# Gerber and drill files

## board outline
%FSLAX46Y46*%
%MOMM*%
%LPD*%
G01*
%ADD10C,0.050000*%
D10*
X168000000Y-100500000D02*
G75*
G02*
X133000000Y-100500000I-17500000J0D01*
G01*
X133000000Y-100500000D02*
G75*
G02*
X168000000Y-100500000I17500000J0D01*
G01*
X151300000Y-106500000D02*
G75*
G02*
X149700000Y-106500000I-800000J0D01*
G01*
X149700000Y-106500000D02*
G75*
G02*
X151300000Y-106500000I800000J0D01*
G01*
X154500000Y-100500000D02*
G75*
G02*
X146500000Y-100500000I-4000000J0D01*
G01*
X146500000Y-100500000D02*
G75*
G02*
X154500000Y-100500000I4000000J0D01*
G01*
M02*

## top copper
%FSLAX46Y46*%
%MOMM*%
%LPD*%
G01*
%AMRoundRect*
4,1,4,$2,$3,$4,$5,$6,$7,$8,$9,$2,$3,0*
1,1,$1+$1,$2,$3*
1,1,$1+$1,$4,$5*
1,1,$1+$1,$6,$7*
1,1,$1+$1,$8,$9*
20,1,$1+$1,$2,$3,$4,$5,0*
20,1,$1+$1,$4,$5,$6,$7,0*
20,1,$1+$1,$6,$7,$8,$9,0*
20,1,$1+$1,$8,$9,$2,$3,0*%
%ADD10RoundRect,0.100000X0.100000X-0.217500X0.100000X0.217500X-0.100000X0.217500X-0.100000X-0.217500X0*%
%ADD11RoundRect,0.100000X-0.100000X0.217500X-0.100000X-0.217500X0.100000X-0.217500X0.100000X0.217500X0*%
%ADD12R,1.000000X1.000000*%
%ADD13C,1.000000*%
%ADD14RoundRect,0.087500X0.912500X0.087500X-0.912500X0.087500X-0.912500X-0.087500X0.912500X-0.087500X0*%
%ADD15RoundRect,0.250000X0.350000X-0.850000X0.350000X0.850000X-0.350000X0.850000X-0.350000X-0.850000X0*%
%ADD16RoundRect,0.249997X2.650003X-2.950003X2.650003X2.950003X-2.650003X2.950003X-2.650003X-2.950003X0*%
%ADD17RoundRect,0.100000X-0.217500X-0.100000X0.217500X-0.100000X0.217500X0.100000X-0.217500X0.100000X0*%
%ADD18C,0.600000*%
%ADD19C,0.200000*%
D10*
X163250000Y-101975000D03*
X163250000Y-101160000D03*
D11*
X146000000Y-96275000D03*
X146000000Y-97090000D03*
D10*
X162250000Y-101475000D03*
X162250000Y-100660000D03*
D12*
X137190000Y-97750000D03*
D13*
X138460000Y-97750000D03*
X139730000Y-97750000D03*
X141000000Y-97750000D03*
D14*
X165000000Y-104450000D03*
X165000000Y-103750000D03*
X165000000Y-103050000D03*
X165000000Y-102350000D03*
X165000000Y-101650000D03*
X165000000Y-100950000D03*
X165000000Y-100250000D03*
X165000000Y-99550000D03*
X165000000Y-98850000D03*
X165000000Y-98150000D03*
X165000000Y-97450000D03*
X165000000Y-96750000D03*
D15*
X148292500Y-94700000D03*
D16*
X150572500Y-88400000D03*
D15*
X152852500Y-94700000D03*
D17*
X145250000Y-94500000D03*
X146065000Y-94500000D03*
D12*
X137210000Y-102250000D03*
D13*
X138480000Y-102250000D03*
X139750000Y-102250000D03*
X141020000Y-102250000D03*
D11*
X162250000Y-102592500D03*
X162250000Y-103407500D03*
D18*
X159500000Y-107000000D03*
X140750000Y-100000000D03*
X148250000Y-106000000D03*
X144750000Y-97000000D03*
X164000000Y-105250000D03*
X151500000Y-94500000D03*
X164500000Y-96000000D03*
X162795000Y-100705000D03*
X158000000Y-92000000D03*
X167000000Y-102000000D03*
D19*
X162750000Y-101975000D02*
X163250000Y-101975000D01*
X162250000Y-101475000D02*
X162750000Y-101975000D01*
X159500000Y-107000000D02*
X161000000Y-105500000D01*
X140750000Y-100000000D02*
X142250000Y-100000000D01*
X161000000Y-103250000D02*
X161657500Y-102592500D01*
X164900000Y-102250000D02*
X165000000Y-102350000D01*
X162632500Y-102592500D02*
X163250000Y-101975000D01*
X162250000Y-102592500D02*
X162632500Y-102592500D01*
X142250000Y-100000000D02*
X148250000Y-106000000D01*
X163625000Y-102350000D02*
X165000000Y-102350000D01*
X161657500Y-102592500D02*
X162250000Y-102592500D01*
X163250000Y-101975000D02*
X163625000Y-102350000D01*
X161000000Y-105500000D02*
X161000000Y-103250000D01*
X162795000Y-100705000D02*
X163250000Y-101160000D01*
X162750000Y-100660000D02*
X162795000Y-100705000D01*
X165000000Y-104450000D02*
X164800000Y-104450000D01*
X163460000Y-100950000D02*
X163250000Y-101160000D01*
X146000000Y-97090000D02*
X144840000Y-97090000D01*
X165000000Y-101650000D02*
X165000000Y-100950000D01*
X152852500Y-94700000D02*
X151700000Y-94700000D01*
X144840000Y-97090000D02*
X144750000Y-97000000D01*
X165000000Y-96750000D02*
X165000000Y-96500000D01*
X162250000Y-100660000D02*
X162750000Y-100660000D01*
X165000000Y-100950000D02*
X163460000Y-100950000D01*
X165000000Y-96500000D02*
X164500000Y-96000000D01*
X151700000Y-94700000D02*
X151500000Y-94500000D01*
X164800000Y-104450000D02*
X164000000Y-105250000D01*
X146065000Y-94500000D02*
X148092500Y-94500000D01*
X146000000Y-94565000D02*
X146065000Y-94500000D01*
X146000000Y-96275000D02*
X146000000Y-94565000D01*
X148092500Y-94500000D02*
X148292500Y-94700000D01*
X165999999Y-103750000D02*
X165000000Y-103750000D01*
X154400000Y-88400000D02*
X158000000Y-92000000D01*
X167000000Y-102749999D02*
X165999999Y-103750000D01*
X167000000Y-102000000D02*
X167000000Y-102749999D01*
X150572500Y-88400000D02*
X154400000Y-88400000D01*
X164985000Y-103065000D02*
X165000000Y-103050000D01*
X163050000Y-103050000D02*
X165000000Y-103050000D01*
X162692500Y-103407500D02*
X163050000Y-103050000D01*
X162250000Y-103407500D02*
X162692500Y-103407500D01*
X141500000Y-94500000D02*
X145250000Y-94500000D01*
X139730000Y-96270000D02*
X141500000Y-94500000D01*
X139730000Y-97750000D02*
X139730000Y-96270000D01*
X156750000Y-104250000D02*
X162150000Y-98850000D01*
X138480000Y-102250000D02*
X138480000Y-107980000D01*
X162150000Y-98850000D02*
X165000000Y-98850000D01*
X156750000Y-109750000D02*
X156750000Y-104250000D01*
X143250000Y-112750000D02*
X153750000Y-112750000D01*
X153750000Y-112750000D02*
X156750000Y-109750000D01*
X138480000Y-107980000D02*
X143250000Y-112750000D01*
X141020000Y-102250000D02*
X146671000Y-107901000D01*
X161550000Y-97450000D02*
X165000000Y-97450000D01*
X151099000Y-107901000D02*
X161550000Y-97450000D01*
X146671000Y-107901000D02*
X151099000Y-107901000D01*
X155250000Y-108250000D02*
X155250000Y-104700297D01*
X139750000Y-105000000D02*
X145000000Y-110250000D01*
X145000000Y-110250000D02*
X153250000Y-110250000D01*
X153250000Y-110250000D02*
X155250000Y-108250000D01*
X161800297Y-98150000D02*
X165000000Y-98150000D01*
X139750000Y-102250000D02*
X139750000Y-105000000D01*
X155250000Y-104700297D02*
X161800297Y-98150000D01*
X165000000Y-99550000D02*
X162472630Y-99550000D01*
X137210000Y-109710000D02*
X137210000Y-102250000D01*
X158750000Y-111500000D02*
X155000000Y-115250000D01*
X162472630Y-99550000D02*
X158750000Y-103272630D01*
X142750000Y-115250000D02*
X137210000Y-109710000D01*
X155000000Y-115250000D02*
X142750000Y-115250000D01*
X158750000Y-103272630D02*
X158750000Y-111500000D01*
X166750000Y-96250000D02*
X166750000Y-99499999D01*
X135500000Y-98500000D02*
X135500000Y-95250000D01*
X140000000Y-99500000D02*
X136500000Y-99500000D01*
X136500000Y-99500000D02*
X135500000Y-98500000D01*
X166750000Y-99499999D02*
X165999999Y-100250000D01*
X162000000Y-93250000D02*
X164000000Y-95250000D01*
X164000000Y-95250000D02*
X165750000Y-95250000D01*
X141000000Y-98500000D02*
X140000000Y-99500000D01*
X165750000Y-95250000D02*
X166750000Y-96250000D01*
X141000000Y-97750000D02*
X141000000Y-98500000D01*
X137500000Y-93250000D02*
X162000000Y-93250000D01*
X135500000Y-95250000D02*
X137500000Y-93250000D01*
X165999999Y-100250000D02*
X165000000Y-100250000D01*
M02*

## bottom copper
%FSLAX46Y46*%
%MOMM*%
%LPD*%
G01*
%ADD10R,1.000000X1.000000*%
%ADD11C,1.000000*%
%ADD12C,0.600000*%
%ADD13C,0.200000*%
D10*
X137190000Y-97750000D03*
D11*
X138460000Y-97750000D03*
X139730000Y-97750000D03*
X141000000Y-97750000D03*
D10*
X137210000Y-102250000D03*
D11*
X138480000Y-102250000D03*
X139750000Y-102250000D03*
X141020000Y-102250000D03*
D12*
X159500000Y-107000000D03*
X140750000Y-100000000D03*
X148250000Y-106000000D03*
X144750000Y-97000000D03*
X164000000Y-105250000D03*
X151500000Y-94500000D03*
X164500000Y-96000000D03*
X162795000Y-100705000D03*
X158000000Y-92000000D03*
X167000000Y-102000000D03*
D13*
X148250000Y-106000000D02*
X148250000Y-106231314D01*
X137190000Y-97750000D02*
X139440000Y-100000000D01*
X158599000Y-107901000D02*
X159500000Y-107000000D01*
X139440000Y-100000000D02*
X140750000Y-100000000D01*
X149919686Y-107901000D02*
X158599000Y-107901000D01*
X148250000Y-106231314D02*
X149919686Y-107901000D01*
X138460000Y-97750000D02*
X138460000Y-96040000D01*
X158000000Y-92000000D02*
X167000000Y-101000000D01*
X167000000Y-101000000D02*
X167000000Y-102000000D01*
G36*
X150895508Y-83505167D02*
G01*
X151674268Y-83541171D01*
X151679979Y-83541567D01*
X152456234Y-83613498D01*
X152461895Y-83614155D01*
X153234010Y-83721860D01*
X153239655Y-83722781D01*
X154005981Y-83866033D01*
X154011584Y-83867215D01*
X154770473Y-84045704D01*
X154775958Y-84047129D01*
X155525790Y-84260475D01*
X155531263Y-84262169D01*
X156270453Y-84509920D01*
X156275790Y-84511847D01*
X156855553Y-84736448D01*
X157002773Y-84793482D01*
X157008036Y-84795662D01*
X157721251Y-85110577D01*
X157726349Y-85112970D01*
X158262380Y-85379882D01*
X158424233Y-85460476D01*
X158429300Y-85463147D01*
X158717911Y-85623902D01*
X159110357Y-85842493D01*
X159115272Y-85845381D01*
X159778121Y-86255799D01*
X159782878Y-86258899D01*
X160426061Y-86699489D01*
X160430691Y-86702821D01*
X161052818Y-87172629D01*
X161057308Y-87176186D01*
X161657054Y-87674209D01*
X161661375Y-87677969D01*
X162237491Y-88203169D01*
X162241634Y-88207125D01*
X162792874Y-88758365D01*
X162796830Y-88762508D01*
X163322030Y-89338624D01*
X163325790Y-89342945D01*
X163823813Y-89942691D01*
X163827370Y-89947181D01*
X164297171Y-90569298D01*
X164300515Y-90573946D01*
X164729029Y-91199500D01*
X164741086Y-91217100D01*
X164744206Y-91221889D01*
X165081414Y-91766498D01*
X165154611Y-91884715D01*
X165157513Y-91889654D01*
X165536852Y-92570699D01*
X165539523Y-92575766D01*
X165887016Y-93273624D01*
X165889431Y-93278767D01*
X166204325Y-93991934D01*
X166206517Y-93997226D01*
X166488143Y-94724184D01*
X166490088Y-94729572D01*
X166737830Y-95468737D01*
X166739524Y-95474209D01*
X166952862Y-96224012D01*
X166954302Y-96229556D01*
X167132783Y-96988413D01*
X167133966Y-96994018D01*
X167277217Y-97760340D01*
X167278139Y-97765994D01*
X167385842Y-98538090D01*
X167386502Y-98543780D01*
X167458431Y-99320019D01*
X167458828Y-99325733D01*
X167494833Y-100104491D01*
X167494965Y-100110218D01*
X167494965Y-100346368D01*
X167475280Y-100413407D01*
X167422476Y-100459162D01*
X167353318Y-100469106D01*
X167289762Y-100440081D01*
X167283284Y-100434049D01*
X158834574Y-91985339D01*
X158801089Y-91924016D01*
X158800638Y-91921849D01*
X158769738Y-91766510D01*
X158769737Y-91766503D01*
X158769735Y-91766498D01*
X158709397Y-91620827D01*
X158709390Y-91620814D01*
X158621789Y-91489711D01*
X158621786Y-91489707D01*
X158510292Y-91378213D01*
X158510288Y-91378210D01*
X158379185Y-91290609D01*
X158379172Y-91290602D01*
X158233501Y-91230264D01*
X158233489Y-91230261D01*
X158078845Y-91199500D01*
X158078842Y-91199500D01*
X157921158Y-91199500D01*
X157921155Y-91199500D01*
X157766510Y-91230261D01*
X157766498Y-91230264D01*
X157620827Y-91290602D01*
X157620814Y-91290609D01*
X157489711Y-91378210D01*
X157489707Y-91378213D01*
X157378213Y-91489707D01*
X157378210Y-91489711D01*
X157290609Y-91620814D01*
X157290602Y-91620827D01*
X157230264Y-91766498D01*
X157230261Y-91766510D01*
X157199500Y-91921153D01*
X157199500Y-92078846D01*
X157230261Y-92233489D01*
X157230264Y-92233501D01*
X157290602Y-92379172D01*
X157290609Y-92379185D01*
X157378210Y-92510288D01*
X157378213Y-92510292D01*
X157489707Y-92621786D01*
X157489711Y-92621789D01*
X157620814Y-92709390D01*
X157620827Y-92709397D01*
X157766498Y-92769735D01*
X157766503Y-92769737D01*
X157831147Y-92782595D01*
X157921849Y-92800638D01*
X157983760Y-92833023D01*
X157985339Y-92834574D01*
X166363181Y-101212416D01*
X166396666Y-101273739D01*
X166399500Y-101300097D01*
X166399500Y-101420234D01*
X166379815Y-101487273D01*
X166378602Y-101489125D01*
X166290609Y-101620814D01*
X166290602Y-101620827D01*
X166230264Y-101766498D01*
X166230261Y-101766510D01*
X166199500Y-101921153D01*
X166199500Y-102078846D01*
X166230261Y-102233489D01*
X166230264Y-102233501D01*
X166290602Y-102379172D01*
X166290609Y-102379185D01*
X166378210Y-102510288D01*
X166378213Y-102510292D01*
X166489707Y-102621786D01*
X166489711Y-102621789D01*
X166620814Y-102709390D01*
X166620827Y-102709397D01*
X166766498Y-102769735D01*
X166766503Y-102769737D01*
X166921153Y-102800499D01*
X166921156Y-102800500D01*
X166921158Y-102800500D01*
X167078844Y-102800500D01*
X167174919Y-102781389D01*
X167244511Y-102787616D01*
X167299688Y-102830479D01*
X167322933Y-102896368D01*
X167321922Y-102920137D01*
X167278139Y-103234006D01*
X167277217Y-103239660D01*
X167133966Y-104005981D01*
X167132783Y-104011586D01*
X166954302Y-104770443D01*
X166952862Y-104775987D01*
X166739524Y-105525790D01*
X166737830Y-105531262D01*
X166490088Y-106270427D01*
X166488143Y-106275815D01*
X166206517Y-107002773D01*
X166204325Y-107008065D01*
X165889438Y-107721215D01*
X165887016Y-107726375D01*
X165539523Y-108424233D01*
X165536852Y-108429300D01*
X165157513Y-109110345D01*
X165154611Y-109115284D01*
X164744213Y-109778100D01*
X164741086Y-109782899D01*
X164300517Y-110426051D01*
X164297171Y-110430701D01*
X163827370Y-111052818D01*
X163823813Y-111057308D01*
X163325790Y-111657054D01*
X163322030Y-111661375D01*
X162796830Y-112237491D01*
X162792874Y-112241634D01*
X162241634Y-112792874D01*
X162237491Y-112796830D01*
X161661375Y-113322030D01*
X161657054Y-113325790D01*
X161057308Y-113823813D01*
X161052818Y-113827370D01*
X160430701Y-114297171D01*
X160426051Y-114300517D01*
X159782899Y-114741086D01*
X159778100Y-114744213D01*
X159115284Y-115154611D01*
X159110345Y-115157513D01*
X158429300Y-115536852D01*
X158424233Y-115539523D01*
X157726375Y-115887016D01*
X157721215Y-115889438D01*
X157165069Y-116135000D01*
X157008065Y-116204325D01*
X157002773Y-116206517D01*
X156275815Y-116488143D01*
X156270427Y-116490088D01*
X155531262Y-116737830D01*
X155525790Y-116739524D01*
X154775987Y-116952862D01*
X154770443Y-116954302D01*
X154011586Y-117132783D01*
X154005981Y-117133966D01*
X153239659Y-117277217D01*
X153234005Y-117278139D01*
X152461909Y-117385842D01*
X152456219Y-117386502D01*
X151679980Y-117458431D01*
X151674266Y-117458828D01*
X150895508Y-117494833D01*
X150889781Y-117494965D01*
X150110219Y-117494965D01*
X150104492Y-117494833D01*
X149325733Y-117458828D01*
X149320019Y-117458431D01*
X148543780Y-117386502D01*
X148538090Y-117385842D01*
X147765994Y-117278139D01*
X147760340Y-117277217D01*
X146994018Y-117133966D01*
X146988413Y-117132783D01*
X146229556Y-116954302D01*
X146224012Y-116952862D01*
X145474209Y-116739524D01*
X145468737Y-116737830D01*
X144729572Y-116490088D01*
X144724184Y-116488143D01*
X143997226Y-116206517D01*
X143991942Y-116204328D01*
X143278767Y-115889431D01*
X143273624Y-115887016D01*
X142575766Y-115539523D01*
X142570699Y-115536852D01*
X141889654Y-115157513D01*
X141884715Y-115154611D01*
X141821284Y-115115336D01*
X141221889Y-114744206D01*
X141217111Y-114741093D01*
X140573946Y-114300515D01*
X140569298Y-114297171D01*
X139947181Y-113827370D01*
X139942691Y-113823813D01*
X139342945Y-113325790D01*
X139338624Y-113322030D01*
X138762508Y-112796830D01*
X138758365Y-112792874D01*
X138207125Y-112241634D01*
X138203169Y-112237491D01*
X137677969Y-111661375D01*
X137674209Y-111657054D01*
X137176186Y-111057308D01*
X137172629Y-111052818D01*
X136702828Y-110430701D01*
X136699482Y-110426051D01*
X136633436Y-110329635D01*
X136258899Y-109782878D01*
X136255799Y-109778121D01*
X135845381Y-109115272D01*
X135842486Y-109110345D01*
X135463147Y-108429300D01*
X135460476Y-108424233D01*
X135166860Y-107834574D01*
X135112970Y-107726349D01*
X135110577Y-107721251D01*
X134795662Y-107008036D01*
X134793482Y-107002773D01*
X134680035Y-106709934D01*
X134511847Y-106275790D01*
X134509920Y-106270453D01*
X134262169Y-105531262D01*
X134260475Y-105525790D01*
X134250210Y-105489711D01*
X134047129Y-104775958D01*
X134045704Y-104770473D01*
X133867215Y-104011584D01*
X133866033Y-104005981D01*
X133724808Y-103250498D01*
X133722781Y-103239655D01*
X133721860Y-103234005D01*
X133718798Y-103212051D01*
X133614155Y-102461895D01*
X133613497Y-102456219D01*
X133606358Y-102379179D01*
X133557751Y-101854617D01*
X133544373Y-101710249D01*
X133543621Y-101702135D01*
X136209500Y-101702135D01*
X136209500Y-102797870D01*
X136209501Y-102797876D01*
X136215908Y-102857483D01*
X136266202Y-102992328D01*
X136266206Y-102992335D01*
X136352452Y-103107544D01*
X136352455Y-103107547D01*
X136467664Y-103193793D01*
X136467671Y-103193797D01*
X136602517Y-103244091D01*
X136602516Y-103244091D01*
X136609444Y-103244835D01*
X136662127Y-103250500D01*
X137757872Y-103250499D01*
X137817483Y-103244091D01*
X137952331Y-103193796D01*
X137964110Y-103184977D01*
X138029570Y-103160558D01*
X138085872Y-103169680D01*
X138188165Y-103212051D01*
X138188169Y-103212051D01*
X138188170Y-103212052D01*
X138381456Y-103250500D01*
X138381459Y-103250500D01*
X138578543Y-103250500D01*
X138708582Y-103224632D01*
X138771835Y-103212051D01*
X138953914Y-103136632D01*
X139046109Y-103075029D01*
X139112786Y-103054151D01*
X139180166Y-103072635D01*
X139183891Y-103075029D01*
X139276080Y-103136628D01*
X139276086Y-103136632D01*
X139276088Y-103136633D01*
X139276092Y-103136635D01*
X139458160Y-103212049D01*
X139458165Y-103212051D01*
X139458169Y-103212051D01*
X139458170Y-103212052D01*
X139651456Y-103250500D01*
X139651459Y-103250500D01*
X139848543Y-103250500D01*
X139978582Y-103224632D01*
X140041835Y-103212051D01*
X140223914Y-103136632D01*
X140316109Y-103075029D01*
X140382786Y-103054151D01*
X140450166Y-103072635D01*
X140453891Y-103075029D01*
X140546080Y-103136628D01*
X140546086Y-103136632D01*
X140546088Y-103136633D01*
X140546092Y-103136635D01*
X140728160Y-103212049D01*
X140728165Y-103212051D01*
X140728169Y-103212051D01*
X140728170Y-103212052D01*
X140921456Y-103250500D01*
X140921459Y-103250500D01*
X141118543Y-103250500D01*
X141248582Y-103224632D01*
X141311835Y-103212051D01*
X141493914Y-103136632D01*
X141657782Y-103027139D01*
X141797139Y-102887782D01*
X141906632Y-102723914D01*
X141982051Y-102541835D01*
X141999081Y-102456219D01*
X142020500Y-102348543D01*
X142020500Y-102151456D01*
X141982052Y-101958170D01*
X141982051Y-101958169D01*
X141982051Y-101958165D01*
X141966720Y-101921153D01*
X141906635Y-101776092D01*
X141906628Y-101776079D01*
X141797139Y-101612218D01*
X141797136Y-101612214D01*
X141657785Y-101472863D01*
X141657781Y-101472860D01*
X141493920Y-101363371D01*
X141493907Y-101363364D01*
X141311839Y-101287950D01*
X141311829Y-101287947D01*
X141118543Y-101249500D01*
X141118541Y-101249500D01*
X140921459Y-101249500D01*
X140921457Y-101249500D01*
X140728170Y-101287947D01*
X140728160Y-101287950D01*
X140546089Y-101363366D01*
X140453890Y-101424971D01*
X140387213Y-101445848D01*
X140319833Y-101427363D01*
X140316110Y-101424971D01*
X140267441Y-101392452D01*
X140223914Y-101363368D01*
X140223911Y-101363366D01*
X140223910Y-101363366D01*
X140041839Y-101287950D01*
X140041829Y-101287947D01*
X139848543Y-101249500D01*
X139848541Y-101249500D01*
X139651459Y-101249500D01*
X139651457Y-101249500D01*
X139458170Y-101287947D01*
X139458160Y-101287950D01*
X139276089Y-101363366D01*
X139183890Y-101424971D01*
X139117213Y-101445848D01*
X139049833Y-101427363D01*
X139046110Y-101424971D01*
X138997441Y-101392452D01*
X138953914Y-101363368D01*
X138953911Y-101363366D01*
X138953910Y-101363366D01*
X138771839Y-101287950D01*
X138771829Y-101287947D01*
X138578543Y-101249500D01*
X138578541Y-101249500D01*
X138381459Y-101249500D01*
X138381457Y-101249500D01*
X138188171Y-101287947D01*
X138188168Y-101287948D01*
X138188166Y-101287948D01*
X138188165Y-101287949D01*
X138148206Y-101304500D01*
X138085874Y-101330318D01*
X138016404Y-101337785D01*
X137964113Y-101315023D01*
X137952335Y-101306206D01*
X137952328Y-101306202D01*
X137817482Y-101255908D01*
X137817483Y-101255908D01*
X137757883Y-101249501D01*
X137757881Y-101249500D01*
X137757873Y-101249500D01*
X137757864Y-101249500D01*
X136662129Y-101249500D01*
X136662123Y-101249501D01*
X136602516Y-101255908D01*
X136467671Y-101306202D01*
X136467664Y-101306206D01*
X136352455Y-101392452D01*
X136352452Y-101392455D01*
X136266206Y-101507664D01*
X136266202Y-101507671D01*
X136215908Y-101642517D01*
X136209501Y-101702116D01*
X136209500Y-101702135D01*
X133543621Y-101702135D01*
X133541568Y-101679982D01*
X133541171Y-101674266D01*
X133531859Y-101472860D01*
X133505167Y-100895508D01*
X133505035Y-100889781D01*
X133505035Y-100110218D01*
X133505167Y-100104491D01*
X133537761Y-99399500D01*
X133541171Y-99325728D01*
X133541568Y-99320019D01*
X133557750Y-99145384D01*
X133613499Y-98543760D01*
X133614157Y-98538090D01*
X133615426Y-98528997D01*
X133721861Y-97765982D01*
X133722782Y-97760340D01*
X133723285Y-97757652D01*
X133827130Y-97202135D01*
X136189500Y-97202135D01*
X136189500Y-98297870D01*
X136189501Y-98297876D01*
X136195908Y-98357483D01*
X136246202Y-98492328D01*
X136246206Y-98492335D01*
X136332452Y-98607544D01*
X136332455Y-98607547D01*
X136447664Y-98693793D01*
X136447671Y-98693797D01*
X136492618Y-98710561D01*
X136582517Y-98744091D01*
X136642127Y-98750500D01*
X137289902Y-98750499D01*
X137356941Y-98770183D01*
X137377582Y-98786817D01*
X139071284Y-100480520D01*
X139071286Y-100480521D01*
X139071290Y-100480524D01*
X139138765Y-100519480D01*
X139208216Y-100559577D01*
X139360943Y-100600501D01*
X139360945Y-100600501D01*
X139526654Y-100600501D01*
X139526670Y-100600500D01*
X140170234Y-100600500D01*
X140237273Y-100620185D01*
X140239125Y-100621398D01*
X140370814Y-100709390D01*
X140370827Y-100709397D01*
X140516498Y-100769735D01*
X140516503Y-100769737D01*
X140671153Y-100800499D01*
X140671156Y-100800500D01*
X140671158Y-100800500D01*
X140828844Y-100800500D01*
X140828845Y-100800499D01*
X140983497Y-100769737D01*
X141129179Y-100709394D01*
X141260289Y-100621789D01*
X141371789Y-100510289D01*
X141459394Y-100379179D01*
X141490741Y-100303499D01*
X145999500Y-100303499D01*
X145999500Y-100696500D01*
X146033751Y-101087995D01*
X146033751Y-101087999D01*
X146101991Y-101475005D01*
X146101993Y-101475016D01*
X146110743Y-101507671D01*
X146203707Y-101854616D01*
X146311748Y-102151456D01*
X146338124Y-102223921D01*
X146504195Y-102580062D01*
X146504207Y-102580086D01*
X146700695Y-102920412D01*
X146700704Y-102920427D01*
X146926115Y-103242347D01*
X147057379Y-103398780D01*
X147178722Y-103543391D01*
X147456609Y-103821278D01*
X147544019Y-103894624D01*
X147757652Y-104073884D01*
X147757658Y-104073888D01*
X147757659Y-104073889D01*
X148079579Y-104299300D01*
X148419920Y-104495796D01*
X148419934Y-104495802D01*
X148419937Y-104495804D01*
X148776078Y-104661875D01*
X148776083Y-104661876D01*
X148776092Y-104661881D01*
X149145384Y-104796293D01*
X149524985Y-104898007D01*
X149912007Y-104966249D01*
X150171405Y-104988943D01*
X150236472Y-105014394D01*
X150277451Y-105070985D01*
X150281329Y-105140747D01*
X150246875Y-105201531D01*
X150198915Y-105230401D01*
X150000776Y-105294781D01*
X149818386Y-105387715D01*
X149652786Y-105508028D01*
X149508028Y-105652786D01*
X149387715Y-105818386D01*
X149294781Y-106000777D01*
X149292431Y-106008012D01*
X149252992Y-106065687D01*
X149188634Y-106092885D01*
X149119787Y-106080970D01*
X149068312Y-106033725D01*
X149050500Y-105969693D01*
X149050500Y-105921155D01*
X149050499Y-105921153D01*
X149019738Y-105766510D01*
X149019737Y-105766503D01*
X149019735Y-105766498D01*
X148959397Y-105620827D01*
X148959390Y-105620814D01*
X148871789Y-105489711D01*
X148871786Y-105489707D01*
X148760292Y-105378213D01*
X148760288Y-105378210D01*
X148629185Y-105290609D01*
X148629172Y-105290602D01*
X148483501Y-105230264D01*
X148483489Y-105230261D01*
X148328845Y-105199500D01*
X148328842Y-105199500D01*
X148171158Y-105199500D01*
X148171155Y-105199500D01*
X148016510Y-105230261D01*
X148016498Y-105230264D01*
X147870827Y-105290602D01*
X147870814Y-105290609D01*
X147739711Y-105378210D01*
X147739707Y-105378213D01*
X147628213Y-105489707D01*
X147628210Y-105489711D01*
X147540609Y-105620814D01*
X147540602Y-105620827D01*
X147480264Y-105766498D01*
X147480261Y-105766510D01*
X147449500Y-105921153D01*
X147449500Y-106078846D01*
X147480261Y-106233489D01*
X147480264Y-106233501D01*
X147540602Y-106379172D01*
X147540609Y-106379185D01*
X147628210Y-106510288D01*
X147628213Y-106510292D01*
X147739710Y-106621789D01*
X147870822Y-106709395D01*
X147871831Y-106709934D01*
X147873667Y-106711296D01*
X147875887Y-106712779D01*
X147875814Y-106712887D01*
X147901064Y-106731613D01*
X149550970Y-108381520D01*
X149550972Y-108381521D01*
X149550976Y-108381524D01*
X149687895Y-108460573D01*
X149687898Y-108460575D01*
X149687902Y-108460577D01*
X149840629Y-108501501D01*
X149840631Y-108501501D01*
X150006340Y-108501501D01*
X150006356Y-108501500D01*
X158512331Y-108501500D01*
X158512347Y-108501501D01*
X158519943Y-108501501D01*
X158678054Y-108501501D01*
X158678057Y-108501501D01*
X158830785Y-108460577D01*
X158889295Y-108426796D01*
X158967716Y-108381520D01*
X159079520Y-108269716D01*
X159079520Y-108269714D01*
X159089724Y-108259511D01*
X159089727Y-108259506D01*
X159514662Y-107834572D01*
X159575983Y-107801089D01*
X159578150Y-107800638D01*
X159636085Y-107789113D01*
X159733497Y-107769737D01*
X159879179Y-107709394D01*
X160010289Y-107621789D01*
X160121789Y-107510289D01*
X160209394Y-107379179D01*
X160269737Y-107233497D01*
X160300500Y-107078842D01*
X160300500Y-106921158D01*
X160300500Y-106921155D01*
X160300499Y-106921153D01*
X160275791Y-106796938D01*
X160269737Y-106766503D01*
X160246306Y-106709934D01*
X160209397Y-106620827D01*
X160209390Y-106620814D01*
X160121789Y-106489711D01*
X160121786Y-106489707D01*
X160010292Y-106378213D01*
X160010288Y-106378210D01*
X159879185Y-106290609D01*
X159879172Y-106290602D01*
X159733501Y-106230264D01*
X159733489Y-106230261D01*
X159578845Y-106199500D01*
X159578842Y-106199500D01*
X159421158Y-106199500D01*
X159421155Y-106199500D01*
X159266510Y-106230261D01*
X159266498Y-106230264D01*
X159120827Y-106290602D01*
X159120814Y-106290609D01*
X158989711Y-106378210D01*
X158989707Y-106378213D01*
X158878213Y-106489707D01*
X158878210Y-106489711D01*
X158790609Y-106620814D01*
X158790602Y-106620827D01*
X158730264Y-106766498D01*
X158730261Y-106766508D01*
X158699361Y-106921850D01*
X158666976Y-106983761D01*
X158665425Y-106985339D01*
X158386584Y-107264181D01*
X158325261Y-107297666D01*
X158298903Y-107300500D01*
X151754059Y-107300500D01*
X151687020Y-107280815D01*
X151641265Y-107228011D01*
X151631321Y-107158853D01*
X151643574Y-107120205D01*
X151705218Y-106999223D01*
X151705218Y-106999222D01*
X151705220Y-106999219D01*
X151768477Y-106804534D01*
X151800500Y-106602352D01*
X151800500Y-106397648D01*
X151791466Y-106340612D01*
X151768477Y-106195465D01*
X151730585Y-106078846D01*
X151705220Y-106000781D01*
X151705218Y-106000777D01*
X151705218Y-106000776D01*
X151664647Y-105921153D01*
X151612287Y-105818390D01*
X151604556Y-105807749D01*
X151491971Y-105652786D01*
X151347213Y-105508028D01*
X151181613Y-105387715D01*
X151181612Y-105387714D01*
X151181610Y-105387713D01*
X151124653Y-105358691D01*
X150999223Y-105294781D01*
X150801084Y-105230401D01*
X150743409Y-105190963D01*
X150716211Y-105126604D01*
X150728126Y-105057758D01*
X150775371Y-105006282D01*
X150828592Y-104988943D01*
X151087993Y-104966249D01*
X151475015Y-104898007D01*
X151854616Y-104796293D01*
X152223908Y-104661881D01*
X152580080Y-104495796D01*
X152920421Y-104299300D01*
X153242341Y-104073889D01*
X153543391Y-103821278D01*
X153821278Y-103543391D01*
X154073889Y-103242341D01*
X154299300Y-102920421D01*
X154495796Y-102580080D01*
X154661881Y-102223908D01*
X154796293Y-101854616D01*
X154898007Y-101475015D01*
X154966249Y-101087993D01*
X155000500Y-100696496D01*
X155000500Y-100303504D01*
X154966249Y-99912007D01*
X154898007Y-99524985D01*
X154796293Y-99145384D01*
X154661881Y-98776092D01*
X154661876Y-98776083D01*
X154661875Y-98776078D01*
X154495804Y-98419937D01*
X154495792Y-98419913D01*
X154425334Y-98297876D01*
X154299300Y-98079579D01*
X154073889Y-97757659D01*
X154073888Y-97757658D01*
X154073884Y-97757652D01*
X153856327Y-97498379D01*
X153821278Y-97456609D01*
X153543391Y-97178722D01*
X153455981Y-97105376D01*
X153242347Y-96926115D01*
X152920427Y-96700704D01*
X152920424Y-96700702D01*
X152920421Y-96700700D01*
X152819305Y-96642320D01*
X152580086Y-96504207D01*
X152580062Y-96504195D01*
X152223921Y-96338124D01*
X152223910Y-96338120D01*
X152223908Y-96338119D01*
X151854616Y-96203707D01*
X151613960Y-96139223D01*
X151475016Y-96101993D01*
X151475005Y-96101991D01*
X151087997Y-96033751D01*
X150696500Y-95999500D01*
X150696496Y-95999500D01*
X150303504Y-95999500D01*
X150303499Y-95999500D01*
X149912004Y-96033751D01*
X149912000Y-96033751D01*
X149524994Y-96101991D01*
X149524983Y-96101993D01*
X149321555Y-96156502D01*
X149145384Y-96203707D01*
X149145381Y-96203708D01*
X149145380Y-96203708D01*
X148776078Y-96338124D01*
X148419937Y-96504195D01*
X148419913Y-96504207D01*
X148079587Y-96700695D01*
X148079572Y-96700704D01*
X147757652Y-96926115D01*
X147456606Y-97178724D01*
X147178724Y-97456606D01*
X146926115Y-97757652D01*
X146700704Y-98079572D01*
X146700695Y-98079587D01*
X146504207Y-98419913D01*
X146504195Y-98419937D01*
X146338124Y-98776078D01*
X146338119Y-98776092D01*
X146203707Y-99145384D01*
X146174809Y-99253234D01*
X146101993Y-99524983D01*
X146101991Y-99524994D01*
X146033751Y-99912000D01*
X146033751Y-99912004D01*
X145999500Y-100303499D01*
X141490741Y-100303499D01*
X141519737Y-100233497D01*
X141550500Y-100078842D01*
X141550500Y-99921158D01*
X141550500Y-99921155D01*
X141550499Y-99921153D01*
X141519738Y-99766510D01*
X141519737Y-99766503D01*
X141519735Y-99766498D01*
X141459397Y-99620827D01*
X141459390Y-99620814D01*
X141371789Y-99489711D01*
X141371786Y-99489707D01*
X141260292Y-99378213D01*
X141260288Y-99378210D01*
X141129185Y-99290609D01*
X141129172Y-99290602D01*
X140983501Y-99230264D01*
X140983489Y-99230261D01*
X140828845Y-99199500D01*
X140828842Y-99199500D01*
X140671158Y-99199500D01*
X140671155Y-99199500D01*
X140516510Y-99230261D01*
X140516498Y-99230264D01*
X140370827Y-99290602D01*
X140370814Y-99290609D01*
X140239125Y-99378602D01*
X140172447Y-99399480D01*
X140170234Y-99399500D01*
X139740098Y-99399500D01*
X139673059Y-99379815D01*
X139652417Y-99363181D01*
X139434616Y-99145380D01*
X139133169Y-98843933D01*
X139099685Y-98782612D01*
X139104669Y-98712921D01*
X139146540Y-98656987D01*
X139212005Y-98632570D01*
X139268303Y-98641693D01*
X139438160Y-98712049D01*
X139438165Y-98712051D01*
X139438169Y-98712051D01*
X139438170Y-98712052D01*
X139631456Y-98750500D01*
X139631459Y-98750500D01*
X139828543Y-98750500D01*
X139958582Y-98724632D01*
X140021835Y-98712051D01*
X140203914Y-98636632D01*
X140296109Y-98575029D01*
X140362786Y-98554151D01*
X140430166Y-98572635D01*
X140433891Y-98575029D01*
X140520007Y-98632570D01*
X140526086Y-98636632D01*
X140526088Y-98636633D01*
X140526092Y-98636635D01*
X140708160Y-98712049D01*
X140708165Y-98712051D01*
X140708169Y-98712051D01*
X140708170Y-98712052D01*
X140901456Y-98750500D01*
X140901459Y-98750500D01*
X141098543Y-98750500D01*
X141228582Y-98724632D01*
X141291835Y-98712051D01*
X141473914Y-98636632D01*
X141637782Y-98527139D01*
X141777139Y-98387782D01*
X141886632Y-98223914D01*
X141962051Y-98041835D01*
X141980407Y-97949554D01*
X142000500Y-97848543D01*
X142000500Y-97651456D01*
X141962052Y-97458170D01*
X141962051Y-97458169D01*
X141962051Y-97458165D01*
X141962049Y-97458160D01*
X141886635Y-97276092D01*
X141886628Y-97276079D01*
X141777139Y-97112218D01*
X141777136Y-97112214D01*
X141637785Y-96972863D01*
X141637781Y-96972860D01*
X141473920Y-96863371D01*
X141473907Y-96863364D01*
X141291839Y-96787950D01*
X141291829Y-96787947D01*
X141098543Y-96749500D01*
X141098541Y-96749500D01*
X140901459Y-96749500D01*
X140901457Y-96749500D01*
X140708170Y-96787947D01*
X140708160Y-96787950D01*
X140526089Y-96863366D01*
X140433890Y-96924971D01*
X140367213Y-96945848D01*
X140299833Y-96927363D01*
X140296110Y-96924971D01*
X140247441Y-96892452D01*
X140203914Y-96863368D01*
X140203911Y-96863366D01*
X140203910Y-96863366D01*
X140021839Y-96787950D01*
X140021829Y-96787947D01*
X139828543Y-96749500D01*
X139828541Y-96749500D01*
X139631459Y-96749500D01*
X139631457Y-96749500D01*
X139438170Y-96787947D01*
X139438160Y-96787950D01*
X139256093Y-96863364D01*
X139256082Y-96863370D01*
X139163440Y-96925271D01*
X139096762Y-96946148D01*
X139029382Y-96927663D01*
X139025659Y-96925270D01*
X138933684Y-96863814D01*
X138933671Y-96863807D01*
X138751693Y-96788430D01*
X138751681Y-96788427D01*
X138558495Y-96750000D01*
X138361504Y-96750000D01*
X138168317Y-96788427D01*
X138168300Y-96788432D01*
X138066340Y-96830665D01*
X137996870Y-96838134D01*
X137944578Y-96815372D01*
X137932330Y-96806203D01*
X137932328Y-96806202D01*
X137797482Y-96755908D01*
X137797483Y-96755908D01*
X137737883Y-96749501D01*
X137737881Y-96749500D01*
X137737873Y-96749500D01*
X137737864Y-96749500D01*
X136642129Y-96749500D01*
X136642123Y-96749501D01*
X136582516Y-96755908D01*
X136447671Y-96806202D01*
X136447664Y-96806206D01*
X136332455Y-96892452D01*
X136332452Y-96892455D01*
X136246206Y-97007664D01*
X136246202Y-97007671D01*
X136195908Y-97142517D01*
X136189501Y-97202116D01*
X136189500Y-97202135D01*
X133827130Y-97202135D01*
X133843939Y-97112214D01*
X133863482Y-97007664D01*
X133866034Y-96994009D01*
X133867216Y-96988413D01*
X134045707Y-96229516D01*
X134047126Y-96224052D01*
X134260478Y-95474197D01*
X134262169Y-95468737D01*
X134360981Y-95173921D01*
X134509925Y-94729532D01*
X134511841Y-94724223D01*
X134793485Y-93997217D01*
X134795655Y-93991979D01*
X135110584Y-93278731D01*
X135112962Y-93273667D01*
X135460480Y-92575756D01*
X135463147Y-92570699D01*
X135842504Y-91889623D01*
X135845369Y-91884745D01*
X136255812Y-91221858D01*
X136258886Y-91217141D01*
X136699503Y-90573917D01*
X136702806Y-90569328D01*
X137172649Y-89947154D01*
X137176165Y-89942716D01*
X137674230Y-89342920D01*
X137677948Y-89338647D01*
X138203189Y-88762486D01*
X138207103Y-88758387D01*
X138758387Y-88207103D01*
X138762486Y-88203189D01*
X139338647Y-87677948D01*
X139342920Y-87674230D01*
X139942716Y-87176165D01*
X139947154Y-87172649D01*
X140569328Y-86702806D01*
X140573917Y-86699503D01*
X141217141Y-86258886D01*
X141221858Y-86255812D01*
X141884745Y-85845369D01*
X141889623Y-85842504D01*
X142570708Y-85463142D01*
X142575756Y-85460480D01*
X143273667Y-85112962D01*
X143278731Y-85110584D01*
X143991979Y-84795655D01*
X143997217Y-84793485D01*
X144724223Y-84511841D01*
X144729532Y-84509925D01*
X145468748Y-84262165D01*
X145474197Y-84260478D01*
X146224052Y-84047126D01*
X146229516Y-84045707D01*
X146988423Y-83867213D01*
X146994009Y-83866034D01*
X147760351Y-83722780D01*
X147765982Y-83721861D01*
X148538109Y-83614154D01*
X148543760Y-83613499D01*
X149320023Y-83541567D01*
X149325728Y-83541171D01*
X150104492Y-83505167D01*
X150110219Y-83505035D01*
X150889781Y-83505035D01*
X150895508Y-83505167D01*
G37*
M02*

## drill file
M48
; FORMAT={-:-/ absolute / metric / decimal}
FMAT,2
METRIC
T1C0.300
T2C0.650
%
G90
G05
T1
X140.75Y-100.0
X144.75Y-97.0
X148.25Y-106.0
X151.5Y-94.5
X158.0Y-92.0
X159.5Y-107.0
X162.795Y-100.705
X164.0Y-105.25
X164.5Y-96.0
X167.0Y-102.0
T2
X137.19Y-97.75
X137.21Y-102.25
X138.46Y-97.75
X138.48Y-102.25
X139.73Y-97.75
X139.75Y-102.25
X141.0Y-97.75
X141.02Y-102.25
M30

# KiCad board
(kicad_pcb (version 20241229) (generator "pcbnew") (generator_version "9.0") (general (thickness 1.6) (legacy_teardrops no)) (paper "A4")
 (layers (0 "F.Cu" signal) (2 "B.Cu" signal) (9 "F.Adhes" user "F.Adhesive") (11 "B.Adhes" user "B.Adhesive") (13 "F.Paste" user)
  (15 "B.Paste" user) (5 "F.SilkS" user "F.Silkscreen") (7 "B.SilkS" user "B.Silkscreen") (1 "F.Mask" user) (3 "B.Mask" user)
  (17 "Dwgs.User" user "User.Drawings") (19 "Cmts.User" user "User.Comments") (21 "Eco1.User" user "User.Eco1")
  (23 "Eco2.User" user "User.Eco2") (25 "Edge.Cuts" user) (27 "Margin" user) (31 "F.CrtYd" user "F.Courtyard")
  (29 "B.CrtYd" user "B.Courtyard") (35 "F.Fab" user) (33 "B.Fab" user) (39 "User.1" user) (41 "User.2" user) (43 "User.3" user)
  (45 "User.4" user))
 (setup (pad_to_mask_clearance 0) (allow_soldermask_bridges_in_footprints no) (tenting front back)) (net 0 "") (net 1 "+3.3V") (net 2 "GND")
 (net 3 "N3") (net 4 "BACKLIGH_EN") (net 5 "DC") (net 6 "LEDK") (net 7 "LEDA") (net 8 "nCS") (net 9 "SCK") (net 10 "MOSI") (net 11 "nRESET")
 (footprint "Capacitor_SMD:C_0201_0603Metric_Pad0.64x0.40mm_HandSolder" (layer "F.Cu") (at 163.25 101.5675 90)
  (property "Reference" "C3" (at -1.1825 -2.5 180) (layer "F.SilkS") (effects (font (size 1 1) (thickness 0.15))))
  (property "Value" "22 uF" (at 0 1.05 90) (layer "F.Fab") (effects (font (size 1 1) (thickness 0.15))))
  (pad "" smd roundrect (at -0.4325 0 90) (size 0.458 0.36) (layers "F.Paste") (roundrect_rratio 0.25))
  (pad "" smd roundrect (at 0.4325 0 90) (size 0.458 0.36) (layers "F.Paste") (roundrect_rratio 0.25))
  (pad "1" smd roundrect (at -0.4075 0 90) (size 0.635 0.4) (layers "F.Cu" "F.Mask") (roundrect_rratio 0.25) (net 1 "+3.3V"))
  (pad "2" smd roundrect (at 0.4075 0 90) (size 0.635 0.4) (layers "F.Cu" "F.Mask") (roundrect_rratio 0.25) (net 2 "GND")))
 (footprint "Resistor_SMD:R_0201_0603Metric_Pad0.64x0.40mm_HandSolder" (layer "F.Cu") (at 146 96.6825 -90)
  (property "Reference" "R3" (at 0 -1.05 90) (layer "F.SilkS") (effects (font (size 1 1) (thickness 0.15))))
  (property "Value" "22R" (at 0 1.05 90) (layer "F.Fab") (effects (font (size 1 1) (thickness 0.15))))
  (pad "" smd roundrect (at -0.4325 0 270) (size 0.458 0.36) (layers "F.Paste") (roundrect_rratio 0.25))
  (pad "" smd roundrect (at 0.4325 0 270) (size 0.458 0.36) (layers "F.Paste") (roundrect_rratio 0.25))
  (pad "1" smd roundrect (at -0.4075 0 270) (size 0.635 0.4) (layers "F.Cu" "F.Mask") (roundrect_rratio 0.25) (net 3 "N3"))
  (pad "2" smd roundrect (at 0.4075 0 270) (size 0.635 0.4) (layers "F.Cu" "F.Mask") (roundrect_rratio 0.25) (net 2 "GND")))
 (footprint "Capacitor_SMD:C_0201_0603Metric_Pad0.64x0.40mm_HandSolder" (layer "F.Cu") (at 162.25 101.0675 90)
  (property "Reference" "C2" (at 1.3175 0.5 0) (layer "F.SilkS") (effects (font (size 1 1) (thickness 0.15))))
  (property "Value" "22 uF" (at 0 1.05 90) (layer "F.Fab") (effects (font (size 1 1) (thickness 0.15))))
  (pad "" smd roundrect (at -0.4325 0 90) (size 0.458 0.36) (layers "F.Paste") (roundrect_rratio 0.25))
  (pad "" smd roundrect (at 0.4325 0 90) (size 0.458 0.36) (layers "F.Paste") (roundrect_rratio 0.25))
  (pad "1" smd roundrect (at -0.4075 0 90) (size 0.635 0.4) (layers "F.Cu" "F.Mask") (roundrect_rratio 0.25) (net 1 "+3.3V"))
  (pad "2" smd roundrect (at 0.4075 0 90) (size 0.635 0.4) (layers "F.Cu" "F.Mask") (roundrect_rratio 0.25) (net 2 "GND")))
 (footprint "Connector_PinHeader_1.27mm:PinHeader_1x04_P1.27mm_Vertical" (layer "F.Cu") (at 137.19 97.75 90)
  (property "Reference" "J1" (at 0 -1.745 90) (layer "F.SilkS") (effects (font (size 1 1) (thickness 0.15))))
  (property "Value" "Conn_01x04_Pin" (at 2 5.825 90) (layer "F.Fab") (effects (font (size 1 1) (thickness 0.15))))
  (pad "1" thru_hole rect (at 0 0 90) (size 1 1) (drill 0.65) (layers "*.Cu" "*.Mask") (remove_unused_layers no) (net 1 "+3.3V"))
  (pad "2" thru_hole circle (at 0 1.27 90) (size 1 1) (drill 0.65) (layers "*.Cu" "*.Mask") (remove_unused_layers no) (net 2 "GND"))
  (pad "3" thru_hole circle (at 0 2.54 90) (size 1 1) (drill 0.65) (layers "*.Cu" "*.Mask") (remove_unused_layers no) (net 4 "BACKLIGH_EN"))
  (pad "4" thru_hole circle (at 0 3.81 90) (size 1 1) (drill 0.65) (layers "*.Cu" "*.Mask") (remove_unused_layers no) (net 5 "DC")))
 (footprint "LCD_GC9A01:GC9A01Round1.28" (layer "F.Cu") (at 165 100.6 180)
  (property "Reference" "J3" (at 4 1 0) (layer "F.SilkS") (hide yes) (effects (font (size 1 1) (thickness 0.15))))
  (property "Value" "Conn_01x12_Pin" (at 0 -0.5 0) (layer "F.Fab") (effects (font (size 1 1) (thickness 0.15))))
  (pad "1" smd roundrect (at 0 -3.85 180) (size 2 0.35) (layers "F.Cu" "F.Mask" "F.Paste") (roundrect_rratio 0.25) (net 2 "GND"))
  (pad "2" smd roundrect (at 0 -3.15 180) (size 2 0.35) (layers "F.Cu" "F.Mask" "F.Paste") (roundrect_rratio 0.25) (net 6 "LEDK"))
  (pad "3" smd roundrect (at 0 -2.45 180) (size 2 0.35) (layers "F.Cu" "F.Mask" "F.Paste") (roundrect_rratio 0.25) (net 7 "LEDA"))
  (pad "4" smd roundrect (at 0 -1.75 180) (size 2 0.35) (layers "F.Cu" "F.Mask" "F.Paste") (roundrect_rratio 0.25) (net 1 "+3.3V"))
  (pad "5" smd roundrect (at 0 -1.05 180) (size 2 0.35) (layers "F.Cu" "F.Mask" "F.Paste") (roundrect_rratio 0.25) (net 2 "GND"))
  (pad "6" smd roundrect (at 0 -0.35 180) (size 2 0.35) (layers "F.Cu" "F.Mask" "F.Paste") (roundrect_rratio 0.25) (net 2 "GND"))
  (pad "7" smd roundrect (at 0 0.35 180) (size 2 0.35) (layers "F.Cu" "F.Mask" "F.Paste") (roundrect_rratio 0.25) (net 5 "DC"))
  (pad "8" smd roundrect (at 0 1.05 180) (size 2 0.35) (layers "F.Cu" "F.Mask" "F.Paste") (roundrect_rratio 0.25) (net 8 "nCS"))
  (pad "9" smd roundrect (at 0 1.75 180) (size 2 0.35) (layers "F.Cu" "F.Mask" "F.Paste") (roundrect_rratio 0.25) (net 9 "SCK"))
  (pad "10" smd roundrect (at 0 2.45 180) (size 2 0.35) (layers "F.Cu" "F.Mask" "F.Paste") (roundrect_rratio 0.25) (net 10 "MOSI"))
  (pad "11" smd roundrect (at 0 3.15 180) (size 2 0.35) (layers "F.Cu" "F.Mask" "F.Paste") (roundrect_rratio 0.25) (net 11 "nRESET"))
  (pad "12" smd roundrect (at 0 3.85 180) (size 2 0.35) (layers "F.Cu" "F.Mask" "F.Paste") (roundrect_rratio 0.25) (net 2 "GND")))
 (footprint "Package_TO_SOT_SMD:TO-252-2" (layer "F.Cu") (at 150.5725 89.66 90)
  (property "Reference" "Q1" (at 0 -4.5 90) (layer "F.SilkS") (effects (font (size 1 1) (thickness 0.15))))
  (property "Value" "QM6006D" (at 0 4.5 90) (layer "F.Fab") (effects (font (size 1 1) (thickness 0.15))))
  (pad "" smd roundrect (at -0.415 -1.525 90) (size 3.05 2.75) (layers "F.Paste") (roundrect_rratio 0.090909))
  (pad "" smd roundrect (at -0.415 1.525 90) (size 3.05 2.75) (layers "F.Paste") (roundrect_rratio 0.090909))
  (pad "" smd roundrect (at 2.935 -1.525 90) (size 3.05 2.75) (layers "F.Paste") (roundrect_rratio 0.090909))
  (pad "" smd roundrect (at 2.935 1.525 90) (size 3.05 2.75) (layers "F.Paste") (roundrect_rratio 0.090909))
  (pad "1" smd roundrect (at -5.04 -2.28 90) (size 2.2 1.2) (layers "F.Cu" "F.Mask" "F.Paste") (roundrect_rratio 0.208333) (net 3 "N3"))
  (pad "2" smd roundrect (at 1.26 0 90) (size 6.4 5.8) (layers "F.Cu" "F.Mask") (roundrect_rratio 0.043103) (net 6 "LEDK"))
  (pad "3" smd roundrect (at -5.04 2.28 90) (size 2.2 1.2) (layers "F.Cu" "F.Mask" "F.Paste") (roundrect_rratio 0.208333) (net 2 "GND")))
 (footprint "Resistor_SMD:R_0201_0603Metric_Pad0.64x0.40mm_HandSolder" (layer "F.Cu") (at 145.6575 94.5)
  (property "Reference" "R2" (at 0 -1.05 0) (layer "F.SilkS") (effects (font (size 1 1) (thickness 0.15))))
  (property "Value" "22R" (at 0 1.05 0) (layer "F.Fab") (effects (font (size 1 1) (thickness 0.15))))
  (pad "" smd roundrect (at -0.4325 0) (size 0.458 0.36) (layers "F.Paste") (roundrect_rratio 0.25))
  (pad "" smd roundrect (at 0.4325 0) (size 0.458 0.36) (layers "F.Paste") (roundrect_rratio 0.25))
  (pad "1" smd roundrect (at -0.4075 0) (size 0.635 0.4) (layers "F.Cu" "F.Mask") (roundrect_rratio 0.25) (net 4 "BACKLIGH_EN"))
  (pad "2" smd roundrect (at 0.4075 0) (size 0.635 0.4) (layers "F.Cu" "F.Mask") (roundrect_rratio 0.25) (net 3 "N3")))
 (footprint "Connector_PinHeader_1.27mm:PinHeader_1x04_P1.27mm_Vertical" (layer "F.Cu") (at 137.21 102.25 90)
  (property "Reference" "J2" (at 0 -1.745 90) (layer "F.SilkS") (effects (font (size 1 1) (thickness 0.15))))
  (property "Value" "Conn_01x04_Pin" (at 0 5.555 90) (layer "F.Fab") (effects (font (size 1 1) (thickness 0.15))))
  (pad "1" thru_hole rect (at 0 0 90) (size 1 1) (drill 0.65) (layers "*.Cu" "*.Mask") (remove_unused_layers no) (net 8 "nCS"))
  (pad "2" thru_hole circle (at 0 1.27 90) (size 1 1) (drill 0.65) (layers "*.Cu" "*.Mask") (remove_unused_layers no) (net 9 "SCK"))
  (pad "3" thru_hole circle (at 0 2.54 90) (size 1 1) (drill 0.65) (layers "*.Cu" "*.Mask") (remove_unused_layers no) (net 10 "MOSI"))
  (pad "4" thru_hole circle (at 0 3.81 90) (size 1 1) (drill 0.65) (layers "*.Cu" "*.Mask") (remove_unused_layers no) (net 11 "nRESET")))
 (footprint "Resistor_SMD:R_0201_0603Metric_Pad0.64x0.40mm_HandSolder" (layer "F.Cu") (at 162.25 103 -90)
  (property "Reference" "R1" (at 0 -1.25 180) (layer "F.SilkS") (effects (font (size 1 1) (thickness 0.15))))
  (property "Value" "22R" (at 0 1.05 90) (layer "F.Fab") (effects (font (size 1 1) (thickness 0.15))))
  (pad "" smd roundrect (at -0.4325 0 270) (size 0.458 0.36) (layers "F.Paste") (roundrect_rratio 0.25))
  (pad "" smd roundrect (at 0.4325 0 270) (size 0.458 0.36) (layers "F.Paste") (roundrect_rratio 0.25))
  (pad "1" smd roundrect (at -0.4075 0 270) (size 0.635 0.4) (layers "F.Cu" "F.Mask") (roundrect_rratio 0.25) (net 1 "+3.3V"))
  (pad "2" smd roundrect (at 0.4075 0 270) (size 0.635 0.4) (layers "F.Cu" "F.Mask") (roundrect_rratio 0.25) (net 7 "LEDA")))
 (gr_circle (center 150.5 100.5) (end 168 100.5) (stroke (width 0.05) (type solid)) (fill no) (layer "Edge.Cuts"))
 (gr_circle (center 150.5 106.5) (end 151.3 106.5) (stroke (width 0.05) (type solid)) (fill no) (layer "Edge.Cuts"))
 (gr_circle (center 150.5 100.5) (end 154.5 100.5) (stroke (width 0.05) (type default)) (fill no) (layer "Edge.Cuts"))
 (segment (start 162.75 101.975) (end 163.25 101.975) (width 0.2) (layer "F.Cu") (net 1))
 (segment (start 162.25 101.475) (end 162.75 101.975) (width 0.2) (layer "F.Cu") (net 1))
 (segment (start 159.5 107) (end 161 105.5) (width 0.2) (layer "F.Cu") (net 1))
 (segment (start 140.75 100) (end 142.25 100) (width 0.2) (layer "F.Cu") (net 1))
 (segment (start 161 103.25) (end 161.6575 102.5925) (width 0.2) (layer "F.Cu") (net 1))
 (segment (start 164.9 102.25) (end 165 102.35) (width 0.2) (layer "F.Cu") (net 1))
 (segment (start 162.6325 102.5925) (end 163.25 101.975) (width 0.2) (layer "F.Cu") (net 1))
 (segment (start 162.25 102.5925) (end 162.6325 102.5925) (width 0.2) (layer "F.Cu") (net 1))
 (segment (start 142.25 100) (end 148.25 106) (width 0.2) (layer "F.Cu") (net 1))
 (segment (start 163.625 102.35) (end 165 102.35) (width 0.2) (layer "F.Cu") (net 1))
 (segment (start 161.6575 102.5925) (end 162.25 102.5925) (width 0.2) (layer "F.Cu") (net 1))
 (segment (start 163.25 101.975) (end 163.625 102.35) (width 0.2) (layer "F.Cu") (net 1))
 (segment (start 161 105.5) (end 161 103.25) (width 0.2) (layer "F.Cu") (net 1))
 (via (at 159.5 107) (size 0.6) (drill 0.3) (layers "F.Cu" "B.Cu") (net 1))
 (via (at 140.75 100) (size 0.6) (drill 0.3) (layers "F.Cu" "B.Cu") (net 1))
 (via (at 148.25 106) (size 0.6) (drill 0.3) (layers "F.Cu" "B.Cu") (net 1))
 (segment (start 148.25 106) (end 148.25 106.231314) (width 0.2) (layer "B.Cu") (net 1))
 (segment (start 137.19 97.75) (end 139.44 100) (width 0.2) (layer "B.Cu") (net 1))
 (segment (start 158.599 107.901) (end 159.5 107) (width 0.2) (layer "B.Cu") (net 1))
 (segment (start 139.44 100) (end 140.75 100) (width 0.2) (layer "B.Cu") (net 1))
 (segment (start 149.919686 107.901) (end 158.599 107.901) (width 0.2) (layer "B.Cu") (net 1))
 (segment (start 148.25 106.231314) (end 149.919686 107.901) (width 0.2) (layer "B.Cu") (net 1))
 (segment (start 162.795 100.705) (end 163.25 101.16) (width 0.2) (layer "F.Cu") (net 2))
 (segment (start 162.75 100.66) (end 162.795 100.705) (width 0.2) (layer "F.Cu") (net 2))
 (segment (start 165 104.45) (end 164.8 104.45) (width 0.2) (layer "F.Cu") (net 2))
 (segment (start 163.46 100.95) (end 163.25 101.16) (width 0.2) (layer "F.Cu") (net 2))
 (segment (start 146 97.09) (end 144.84 97.09) (width 0.2) (layer "F.Cu") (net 2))
 (segment (start 165 101.65) (end 165 100.95) (width 0.2) (layer "F.Cu") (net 2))
 (segment (start 152.8525 94.7) (end 151.7 94.7) (width 0.2) (layer "F.Cu") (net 2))
 (segment (start 144.84 97.09) (end 144.75 97) (width 0.2) (layer "F.Cu") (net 2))
 (segment (start 165 96.75) (end 165 96.5) (width 0.2) (layer "F.Cu") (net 2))
 (segment (start 162.25 100.66) (end 162.75 100.66) (width 0.2) (layer "F.Cu") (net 2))
 (segment (start 165 100.95) (end 163.46 100.95) (width 0.2) (layer "F.Cu") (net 2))
 (segment (start 165 96.5) (end 164.5 96) (width 0.2) (layer "F.Cu") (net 2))
 (segment (start 151.7 94.7) (end 151.5 94.5) (width 0.2) (layer "F.Cu") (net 2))
 (segment (start 164.8 104.45) (end 164 105.25) (width 0.2) (layer "F.Cu") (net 2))
 (via (at 144.75 97) (size 0.6) (drill 0.3) (layers "F.Cu" "B.Cu") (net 2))
 (via (at 164 105.25) (size 0.6) (drill 0.3) (layers "F.Cu" "B.Cu") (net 2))
 (via (at 151.5 94.5) (size 0.6) (drill 0.3) (layers "F.Cu" "B.Cu") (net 2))
 (via (at 164.5 96) (size 0.6) (drill 0.3) (layers "F.Cu" "B.Cu") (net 2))
 (via (at 162.795 100.705) (size 0.6) (drill 0.3) (layers "F.Cu" "B.Cu") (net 2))
 (segment (start 138.46 97.75) (end 138.46 96.04) (width 0.2) (layer "B.Cu") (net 2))
 (segment (start 146.065 94.5) (end 148.0925 94.5) (width 0.2) (layer "F.Cu") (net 3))
 (segment (start 146 94.565) (end 146.065 94.5) (width 0.2) (layer "F.Cu") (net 3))
 (segment (start 146 96.275) (end 146 94.565) (width 0.2) (layer "F.Cu") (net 3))
 (segment (start 148.0925 94.5) (end 148.2925 94.7) (width 0.2) (layer "F.Cu") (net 3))
 (segment (start 165.999999 103.75) (end 165 103.75) (width 0.2) (layer "F.Cu") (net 6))
 (segment (start 154.4 88.4) (end 158 92) (width 0.2) (layer "F.Cu") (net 6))
 (segment (start 167 102.749999) (end 165.999999 103.75) (width 0.2) (layer "F.Cu") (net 6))
 (segment (start 167 102) (end 167 102.749999) (width 0.2) (layer "F.Cu") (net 6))
 (segment (start 150.5725 88.4) (end 154.4 88.4) (width 0.2) (layer "F.Cu") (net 6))
 (via (at 158 92) (size 0.6) (drill 0.3) (layers "F.Cu" "B.Cu") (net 6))
 (via (at 167 102) (size 0.6) (drill 0.3) (layers "F.Cu" "B.Cu") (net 6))
 (segment (start 158 92) (end 167 101) (width 0.2) (layer "B.Cu") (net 6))
 (segment (start 167 101) (end 167 102) (width 0.2) (layer "B.Cu") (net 6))
 (segment (start 164.985 103.065) (end 165 103.05) (width 0.2) (layer "F.Cu") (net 7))
 (segment (start 163.05 103.05) (end 165 103.05) (width 0.2) (layer "F.Cu") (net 7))
 (segment (start 162.6925 103.4075) (end 163.05 103.05) (width 0.2) (layer "F.Cu") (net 7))
 (segment (start 162.25 103.4075) (end 162.6925 103.4075) (width 0.2) (layer "F.Cu") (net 7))
 (segment (start 141.5 94.5) (end 145.25 94.5) (width 0.2) (layer "F.Cu") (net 4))
 (segment (start 139.73 96.27) (end 141.5 94.5) (width 0.2) (layer "F.Cu") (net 4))
 (segment (start 139.73 97.75) (end 139.73 96.27) (width 0.2) (layer "F.Cu") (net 4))
 (segment (start 156.75 104.25) (end 162.15 98.85) (width 0.2) (layer "F.Cu") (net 9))
 (segment (start 138.48 102.25) (end 138.48 107.98) (width 0.2) (layer "F.Cu") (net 9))
 (segment (start 162.15 98.85) (end 165 98.85) (width 0.2) (layer "F.Cu") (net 9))
 (segment (start 156.75 109.75) (end 156.75 104.25) (width 0.2) (layer "F.Cu") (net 9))
 (segment (start 143.25 112.75) (end 153.75 112.75) (width 0.2) (layer "F.Cu") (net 9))
 (segment (start 153.75 112.75) (end 156.75 109.75) (width 0.2) (layer "F.Cu") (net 9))
 (segment (start 138.48 107.98) (end 143.25 112.75) (width 0.2) (layer "F.Cu") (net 9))
 (segment (start 141.02 102.25) (end 146.671 107.901) (width 0.2) (layer "F.Cu") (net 11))
 (segment (start 161.55 97.45) (end 165 97.45) (width 0.2) (layer "F.Cu") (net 11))
 (segment (start 151.099 107.901) (end 161.55 97.45) (width 0.2) (layer "F.Cu") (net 11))
 (segment (start 146.671 107.901) (end 151.099 107.901) (width 0.2) (layer "F.Cu") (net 11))
 (segment (start 155.25 108.25) (end 155.25 104.700297) (width 0.2) (layer "F.Cu") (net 10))
 (segment (start 139.75 105) (end 145 110.25) (width 0.2) (layer "F.Cu") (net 10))
 (segment (start 145 110.25) (end 153.25 110.25) (width 0.2) (layer "F.Cu") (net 10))
 (segment (start 153.25 110.25) (end 155.25 108.25) (width 0.2) (layer "F.Cu") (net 10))
 (segment (start 161.800297 98.15) (end 165 98.15) (width 0.2) (layer "F.Cu") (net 10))
 (segment (start 139.75 102.25) (end 139.75 105) (width 0.2) (layer "F.Cu") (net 10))
 (segment (start 155.25 104.700297) (end 161.800297 98.15) (width 0.2) (layer "F.Cu") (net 10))
 (segment (start 165 99.55) (end 162.47263 99.55) (width 0.2) (layer "F.Cu") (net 8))
 (segment (start 137.21 109.71) (end 137.21 102.25) (width 0.2) (layer "F.Cu") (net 8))
 (segment (start 158.75 111.5) (end 155 115.25) (width 0.2) (layer "F.Cu") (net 8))
 (segment (start 162.47263 99.55) (end 158.75 103.27263) (width 0.2) (layer "F.Cu") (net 8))
 (segment (start 142.75 115.25) (end 137.21 109.71) (width 0.2) (layer "F.Cu") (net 8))
 (segment (start 155 115.25) (end 142.75 115.25) (width 0.2) (layer "F.Cu") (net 8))
 (segment (start 158.75 103.27263) (end 158.75 111.5) (width 0.2) (layer "F.Cu") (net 8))
 (segment (start 166.75 96.25) (end 166.75 99.499999) (width 0.2) (layer "F.Cu") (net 5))
 (segment (start 135.5 98.5) (end 135.5 95.25) (width 0.2) (layer "F.Cu") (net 5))
 (segment (start 140 99.5) (end 136.5 99.5) (width 0.2) (layer "F.Cu") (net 5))
 (segment (start 136.5 99.5) (end 135.5 98.5) (width 0.2) (layer "F.Cu") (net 5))
 (segment (start 166.75 99.499999) (end 165.999999 100.25) (width 0.2) (layer "F.Cu") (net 5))
 (segment (start 162 93.25) (end 164 95.25) (width 0.2) (layer "F.Cu") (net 5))
 (segment (start 164 95.25) (end 165.75 95.25) (width 0.2) (layer "F.Cu") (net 5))
 (segment (start 141 98.5) (end 140 99.5) (width 0.2) (layer "F.Cu") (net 5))
 (segment (start 165.75 95.25) (end 166.75 96.25) (width 0.2) (layer "F.Cu") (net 5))
 (segment (start 141 97.75) (end 141 98.5) (width 0.2) (layer "F.Cu") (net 5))
 (segment (start 137.5 93.25) (end 162 93.25) (width 0.2) (layer "F.Cu") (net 5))
 (segment (start 135.5 95.25) (end 137.5 93.25) (width 0.2) (layer "F.Cu") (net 5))
 (segment (start 165.999999 100.25) (end 165 100.25) (width 0.2) (layer "F.Cu") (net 5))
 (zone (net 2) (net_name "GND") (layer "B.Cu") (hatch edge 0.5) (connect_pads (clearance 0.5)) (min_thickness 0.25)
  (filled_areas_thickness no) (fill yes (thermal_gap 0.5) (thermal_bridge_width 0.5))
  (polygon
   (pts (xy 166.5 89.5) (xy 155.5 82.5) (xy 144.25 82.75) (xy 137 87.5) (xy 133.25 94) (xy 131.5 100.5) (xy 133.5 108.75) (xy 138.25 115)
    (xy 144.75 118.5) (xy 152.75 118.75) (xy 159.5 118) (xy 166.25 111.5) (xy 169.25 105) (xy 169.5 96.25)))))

